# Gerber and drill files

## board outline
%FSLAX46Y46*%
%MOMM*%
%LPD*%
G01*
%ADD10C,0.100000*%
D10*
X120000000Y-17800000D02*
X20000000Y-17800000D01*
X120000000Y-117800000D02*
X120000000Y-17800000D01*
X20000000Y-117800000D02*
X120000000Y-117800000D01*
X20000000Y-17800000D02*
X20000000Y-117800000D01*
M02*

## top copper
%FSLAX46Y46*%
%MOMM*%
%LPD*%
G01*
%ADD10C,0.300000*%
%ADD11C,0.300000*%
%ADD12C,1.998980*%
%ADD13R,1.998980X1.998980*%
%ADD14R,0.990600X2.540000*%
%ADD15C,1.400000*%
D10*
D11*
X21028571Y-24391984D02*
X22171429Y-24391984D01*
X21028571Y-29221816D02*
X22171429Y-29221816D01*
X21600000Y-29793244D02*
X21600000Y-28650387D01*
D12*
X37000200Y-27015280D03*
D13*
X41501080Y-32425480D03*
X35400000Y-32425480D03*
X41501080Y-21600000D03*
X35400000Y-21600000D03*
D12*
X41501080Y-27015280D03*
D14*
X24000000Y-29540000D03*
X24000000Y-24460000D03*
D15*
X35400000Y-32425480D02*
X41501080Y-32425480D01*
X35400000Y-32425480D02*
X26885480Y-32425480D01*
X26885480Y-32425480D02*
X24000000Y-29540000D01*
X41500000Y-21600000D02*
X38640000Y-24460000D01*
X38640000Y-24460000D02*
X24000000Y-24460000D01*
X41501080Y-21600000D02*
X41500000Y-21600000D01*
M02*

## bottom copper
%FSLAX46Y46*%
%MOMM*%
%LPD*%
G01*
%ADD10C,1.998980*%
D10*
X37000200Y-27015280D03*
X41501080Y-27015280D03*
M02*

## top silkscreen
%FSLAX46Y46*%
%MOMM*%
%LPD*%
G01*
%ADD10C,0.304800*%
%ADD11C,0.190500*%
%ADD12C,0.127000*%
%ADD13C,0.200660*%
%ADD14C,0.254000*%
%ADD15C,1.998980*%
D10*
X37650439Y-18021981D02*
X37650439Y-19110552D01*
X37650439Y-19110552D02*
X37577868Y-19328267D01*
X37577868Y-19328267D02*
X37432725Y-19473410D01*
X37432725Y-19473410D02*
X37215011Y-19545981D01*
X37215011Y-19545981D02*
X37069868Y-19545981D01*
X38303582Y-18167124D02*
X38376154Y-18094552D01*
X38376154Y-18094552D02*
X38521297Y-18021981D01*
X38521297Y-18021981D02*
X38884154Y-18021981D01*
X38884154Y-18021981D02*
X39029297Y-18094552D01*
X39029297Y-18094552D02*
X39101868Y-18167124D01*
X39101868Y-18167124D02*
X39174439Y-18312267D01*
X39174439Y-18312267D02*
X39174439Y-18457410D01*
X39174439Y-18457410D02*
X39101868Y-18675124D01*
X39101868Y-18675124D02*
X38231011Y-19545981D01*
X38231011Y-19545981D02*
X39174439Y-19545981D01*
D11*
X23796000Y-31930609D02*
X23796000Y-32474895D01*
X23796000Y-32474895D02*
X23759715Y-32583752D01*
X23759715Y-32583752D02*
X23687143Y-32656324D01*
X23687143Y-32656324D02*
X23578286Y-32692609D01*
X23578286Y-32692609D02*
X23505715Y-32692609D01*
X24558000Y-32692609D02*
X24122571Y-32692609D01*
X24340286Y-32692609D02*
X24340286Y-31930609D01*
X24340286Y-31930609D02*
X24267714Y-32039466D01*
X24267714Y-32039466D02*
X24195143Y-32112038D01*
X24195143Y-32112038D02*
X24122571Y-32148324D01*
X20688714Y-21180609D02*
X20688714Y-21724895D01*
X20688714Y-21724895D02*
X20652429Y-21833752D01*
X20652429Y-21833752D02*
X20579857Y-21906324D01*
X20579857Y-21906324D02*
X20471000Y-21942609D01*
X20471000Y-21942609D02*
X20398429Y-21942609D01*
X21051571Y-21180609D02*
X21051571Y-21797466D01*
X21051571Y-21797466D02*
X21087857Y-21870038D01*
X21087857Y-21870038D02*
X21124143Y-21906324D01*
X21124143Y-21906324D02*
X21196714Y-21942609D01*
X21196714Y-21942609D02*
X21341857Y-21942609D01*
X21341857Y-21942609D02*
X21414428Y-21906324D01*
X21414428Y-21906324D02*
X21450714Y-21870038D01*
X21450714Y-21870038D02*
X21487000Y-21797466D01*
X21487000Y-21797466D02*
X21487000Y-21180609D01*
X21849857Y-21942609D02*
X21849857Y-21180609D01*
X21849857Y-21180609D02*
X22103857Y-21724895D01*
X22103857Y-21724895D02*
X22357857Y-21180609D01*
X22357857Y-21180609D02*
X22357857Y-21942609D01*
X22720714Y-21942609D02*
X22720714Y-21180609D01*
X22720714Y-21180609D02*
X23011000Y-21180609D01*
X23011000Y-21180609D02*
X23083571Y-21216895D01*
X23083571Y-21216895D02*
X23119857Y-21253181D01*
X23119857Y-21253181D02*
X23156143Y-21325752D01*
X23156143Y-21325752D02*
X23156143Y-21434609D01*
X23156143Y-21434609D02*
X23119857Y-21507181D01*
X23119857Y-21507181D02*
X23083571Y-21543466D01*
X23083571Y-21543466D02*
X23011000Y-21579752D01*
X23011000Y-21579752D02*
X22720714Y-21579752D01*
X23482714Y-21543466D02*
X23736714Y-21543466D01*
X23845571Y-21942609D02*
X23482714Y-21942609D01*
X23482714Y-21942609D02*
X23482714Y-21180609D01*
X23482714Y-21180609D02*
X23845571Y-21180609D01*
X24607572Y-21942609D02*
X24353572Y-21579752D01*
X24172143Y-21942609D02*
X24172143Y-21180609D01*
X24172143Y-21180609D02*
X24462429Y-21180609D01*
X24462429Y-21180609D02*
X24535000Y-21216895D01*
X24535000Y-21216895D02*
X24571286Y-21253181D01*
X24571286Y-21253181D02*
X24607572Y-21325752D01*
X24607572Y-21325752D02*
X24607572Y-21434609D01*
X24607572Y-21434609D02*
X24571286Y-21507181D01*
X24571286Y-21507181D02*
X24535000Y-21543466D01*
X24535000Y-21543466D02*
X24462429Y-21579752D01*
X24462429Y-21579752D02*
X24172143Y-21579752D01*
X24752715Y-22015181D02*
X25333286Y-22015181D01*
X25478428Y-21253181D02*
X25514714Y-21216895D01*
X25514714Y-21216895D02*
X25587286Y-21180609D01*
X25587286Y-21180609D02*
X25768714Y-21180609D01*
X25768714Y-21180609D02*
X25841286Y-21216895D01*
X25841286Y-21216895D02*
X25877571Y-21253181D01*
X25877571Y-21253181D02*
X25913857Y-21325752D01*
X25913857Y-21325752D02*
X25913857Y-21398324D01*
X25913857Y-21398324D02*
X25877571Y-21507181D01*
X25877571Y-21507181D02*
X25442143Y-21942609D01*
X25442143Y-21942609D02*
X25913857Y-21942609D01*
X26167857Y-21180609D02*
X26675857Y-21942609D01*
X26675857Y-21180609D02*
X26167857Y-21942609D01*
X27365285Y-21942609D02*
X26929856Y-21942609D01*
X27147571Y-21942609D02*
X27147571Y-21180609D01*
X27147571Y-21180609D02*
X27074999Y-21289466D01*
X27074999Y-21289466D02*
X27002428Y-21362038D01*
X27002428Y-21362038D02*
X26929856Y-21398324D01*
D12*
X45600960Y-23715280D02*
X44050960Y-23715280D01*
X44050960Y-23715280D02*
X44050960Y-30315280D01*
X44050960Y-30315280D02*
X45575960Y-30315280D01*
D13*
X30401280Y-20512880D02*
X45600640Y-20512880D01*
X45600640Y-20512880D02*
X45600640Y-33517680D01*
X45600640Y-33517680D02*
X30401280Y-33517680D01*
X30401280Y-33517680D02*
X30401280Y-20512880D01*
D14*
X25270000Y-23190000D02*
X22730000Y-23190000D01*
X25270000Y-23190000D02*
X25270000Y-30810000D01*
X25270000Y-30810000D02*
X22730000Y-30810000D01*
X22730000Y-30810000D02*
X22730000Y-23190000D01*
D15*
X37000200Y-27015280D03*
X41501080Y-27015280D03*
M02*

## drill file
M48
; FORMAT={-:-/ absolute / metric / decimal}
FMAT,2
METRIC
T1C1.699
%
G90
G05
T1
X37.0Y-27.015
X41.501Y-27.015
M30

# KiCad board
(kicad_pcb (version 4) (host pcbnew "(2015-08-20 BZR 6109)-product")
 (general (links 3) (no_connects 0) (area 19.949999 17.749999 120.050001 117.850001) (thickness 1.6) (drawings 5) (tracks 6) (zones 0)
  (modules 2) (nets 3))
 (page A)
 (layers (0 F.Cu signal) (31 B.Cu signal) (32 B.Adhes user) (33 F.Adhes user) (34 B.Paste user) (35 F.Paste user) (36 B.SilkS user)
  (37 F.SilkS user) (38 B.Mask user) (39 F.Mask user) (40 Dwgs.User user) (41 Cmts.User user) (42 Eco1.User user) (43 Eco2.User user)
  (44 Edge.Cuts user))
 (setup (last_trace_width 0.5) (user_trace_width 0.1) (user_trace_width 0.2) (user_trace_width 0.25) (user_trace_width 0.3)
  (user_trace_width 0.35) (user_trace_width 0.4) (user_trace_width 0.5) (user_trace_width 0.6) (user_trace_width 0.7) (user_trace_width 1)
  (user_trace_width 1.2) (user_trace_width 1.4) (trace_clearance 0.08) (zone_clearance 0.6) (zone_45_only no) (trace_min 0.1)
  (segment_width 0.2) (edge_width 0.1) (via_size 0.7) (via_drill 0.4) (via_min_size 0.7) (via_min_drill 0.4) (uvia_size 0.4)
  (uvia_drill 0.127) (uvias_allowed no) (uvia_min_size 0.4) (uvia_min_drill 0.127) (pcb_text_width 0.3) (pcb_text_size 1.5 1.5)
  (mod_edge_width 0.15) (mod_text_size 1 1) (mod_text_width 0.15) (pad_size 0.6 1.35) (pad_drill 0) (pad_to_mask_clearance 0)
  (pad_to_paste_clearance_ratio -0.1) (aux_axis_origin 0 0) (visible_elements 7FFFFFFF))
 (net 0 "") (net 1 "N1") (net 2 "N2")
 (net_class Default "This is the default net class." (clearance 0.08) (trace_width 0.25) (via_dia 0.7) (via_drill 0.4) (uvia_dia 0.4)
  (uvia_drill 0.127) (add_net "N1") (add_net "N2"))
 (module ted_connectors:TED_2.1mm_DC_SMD (layer F.Cu) (at 38.00096 27.01528)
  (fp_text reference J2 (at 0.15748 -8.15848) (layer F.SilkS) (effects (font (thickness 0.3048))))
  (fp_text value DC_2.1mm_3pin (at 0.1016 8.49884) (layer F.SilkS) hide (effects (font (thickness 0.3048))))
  (fp_line (start 7.6 -3.3) (end 6.05 -3.3) (layer F.SilkS) (width 0.127))
  (fp_line (start 6.05 -3.3) (end 6.05 3.3) (layer F.SilkS) (width 0.127))
  (fp_line (start 6.05 3.3) (end 7.575 3.3) (layer F.SilkS) (width 0.127))
  (fp_line (start -7.59968 -6.5024) (end 7.59968 -6.5024) (layer F.SilkS) (width 0.20066))
  (fp_line (start 7.59968 -6.5024) (end 7.59968 6.5024) (layer F.SilkS) (width 0.20066))
  (fp_line (start 7.59968 6.5024) (end -7.59968 6.5024) (layer F.SilkS) (width 0.20066))
  (fp_line (start -7.59968 6.5024) (end -7.59968 -6.5024) (layer F.SilkS) (width 0.20066))
  (pad "" np_thru_hole circle (at -1.00076 0) (size 1.99898 1.99898) (drill 1.69926) (layers *.Cu *.Mask F.SilkS))
  (pad 1 smd rect (at 3.50012 5.4102) (size 1.99898 1.99898) (layers F.Cu F.Paste F.Mask) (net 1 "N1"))
  (pad 1 smd rect (at -2.60096 5.4102) (size 1.99898 1.99898) (layers F.Cu F.Paste F.Mask) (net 1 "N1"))
  (pad 2 smd rect (at 3.50012 -5.41528) (size 1.99898 1.99898) (layers F.Cu F.Paste F.Mask) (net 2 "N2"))
  (pad 3 smd rect (at -2.60096 -5.41528) (size 1.99898 1.99898) (layers F.Cu F.Paste F.Mask))
  (pad "" np_thru_hole circle (at 3.50012 0) (size 1.99898 1.99898) (drill 1.69926) (layers *.Cu *.Mask F.SilkS)))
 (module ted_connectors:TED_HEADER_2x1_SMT (layer F.Cu) (at 24 27)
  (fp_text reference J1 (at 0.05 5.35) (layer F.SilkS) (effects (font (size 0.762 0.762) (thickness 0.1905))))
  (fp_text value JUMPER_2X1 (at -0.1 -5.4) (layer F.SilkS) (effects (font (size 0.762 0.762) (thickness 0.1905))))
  (fp_line (start 1.27 -3.81) (end -1.27 -3.81) (layer F.SilkS) (width 0.254))
  (fp_line (start 1.27 -3.81) (end 1.27 3.81) (layer F.SilkS) (width 0.254))
  (fp_line (start 1.27 3.81) (end -1.27 3.81) (layer F.SilkS) (width 0.254))
  (fp_line (start -1.27 3.81) (end -1.27 -3.81) (layer F.SilkS) (width 0.254))
  (pad 1 smd rect (at 0 2.54) (size 0.9906 2.54) (layers F.Cu F.Paste F.Mask) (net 1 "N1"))
  (pad 2 smd rect (at 0 -2.54) (size 0.9906 2.54) (layers F.Cu F.Paste F.Mask) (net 2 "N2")))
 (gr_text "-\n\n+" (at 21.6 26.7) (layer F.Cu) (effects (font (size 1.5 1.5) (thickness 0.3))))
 (gr_line (start 120 17.8) (end 20 17.8) (angle 90) (layer Edge.Cuts) (width 0.1))
 (gr_line (start 120 117.8) (end 120 17.8) (angle 90) (layer Edge.Cuts) (width 0.1))
 (gr_line (start 20 117.8) (end 120 117.8) (angle 90) (layer Edge.Cuts) (width 0.1))
 (gr_line (start 20 17.8) (end 20 117.8) (angle 90) (layer Edge.Cuts) (width 0.1))
 (segment (start 35.4 32.42548) (end 41.50108 32.42548) (width 1.4) (layer F.Cu) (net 1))
 (segment (start 35.4 32.42548) (end 26.88548 32.42548) (width 1.4) (layer F.Cu) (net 1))
 (segment (start 26.88548 32.42548) (end 24 29.54) (width 1.4) (layer F.Cu) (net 1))
 (segment (start 41.5 21.6) (end 38.64 24.46) (width 1.4) (layer F.Cu) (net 2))
 (segment (start 38.64 24.46) (end 24 24.46) (width 1.4) (layer F.Cu) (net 2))
 (segment (start 41.50108 21.6) (end 41.5 21.6) (width 1.4) (layer F.Cu) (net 2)))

